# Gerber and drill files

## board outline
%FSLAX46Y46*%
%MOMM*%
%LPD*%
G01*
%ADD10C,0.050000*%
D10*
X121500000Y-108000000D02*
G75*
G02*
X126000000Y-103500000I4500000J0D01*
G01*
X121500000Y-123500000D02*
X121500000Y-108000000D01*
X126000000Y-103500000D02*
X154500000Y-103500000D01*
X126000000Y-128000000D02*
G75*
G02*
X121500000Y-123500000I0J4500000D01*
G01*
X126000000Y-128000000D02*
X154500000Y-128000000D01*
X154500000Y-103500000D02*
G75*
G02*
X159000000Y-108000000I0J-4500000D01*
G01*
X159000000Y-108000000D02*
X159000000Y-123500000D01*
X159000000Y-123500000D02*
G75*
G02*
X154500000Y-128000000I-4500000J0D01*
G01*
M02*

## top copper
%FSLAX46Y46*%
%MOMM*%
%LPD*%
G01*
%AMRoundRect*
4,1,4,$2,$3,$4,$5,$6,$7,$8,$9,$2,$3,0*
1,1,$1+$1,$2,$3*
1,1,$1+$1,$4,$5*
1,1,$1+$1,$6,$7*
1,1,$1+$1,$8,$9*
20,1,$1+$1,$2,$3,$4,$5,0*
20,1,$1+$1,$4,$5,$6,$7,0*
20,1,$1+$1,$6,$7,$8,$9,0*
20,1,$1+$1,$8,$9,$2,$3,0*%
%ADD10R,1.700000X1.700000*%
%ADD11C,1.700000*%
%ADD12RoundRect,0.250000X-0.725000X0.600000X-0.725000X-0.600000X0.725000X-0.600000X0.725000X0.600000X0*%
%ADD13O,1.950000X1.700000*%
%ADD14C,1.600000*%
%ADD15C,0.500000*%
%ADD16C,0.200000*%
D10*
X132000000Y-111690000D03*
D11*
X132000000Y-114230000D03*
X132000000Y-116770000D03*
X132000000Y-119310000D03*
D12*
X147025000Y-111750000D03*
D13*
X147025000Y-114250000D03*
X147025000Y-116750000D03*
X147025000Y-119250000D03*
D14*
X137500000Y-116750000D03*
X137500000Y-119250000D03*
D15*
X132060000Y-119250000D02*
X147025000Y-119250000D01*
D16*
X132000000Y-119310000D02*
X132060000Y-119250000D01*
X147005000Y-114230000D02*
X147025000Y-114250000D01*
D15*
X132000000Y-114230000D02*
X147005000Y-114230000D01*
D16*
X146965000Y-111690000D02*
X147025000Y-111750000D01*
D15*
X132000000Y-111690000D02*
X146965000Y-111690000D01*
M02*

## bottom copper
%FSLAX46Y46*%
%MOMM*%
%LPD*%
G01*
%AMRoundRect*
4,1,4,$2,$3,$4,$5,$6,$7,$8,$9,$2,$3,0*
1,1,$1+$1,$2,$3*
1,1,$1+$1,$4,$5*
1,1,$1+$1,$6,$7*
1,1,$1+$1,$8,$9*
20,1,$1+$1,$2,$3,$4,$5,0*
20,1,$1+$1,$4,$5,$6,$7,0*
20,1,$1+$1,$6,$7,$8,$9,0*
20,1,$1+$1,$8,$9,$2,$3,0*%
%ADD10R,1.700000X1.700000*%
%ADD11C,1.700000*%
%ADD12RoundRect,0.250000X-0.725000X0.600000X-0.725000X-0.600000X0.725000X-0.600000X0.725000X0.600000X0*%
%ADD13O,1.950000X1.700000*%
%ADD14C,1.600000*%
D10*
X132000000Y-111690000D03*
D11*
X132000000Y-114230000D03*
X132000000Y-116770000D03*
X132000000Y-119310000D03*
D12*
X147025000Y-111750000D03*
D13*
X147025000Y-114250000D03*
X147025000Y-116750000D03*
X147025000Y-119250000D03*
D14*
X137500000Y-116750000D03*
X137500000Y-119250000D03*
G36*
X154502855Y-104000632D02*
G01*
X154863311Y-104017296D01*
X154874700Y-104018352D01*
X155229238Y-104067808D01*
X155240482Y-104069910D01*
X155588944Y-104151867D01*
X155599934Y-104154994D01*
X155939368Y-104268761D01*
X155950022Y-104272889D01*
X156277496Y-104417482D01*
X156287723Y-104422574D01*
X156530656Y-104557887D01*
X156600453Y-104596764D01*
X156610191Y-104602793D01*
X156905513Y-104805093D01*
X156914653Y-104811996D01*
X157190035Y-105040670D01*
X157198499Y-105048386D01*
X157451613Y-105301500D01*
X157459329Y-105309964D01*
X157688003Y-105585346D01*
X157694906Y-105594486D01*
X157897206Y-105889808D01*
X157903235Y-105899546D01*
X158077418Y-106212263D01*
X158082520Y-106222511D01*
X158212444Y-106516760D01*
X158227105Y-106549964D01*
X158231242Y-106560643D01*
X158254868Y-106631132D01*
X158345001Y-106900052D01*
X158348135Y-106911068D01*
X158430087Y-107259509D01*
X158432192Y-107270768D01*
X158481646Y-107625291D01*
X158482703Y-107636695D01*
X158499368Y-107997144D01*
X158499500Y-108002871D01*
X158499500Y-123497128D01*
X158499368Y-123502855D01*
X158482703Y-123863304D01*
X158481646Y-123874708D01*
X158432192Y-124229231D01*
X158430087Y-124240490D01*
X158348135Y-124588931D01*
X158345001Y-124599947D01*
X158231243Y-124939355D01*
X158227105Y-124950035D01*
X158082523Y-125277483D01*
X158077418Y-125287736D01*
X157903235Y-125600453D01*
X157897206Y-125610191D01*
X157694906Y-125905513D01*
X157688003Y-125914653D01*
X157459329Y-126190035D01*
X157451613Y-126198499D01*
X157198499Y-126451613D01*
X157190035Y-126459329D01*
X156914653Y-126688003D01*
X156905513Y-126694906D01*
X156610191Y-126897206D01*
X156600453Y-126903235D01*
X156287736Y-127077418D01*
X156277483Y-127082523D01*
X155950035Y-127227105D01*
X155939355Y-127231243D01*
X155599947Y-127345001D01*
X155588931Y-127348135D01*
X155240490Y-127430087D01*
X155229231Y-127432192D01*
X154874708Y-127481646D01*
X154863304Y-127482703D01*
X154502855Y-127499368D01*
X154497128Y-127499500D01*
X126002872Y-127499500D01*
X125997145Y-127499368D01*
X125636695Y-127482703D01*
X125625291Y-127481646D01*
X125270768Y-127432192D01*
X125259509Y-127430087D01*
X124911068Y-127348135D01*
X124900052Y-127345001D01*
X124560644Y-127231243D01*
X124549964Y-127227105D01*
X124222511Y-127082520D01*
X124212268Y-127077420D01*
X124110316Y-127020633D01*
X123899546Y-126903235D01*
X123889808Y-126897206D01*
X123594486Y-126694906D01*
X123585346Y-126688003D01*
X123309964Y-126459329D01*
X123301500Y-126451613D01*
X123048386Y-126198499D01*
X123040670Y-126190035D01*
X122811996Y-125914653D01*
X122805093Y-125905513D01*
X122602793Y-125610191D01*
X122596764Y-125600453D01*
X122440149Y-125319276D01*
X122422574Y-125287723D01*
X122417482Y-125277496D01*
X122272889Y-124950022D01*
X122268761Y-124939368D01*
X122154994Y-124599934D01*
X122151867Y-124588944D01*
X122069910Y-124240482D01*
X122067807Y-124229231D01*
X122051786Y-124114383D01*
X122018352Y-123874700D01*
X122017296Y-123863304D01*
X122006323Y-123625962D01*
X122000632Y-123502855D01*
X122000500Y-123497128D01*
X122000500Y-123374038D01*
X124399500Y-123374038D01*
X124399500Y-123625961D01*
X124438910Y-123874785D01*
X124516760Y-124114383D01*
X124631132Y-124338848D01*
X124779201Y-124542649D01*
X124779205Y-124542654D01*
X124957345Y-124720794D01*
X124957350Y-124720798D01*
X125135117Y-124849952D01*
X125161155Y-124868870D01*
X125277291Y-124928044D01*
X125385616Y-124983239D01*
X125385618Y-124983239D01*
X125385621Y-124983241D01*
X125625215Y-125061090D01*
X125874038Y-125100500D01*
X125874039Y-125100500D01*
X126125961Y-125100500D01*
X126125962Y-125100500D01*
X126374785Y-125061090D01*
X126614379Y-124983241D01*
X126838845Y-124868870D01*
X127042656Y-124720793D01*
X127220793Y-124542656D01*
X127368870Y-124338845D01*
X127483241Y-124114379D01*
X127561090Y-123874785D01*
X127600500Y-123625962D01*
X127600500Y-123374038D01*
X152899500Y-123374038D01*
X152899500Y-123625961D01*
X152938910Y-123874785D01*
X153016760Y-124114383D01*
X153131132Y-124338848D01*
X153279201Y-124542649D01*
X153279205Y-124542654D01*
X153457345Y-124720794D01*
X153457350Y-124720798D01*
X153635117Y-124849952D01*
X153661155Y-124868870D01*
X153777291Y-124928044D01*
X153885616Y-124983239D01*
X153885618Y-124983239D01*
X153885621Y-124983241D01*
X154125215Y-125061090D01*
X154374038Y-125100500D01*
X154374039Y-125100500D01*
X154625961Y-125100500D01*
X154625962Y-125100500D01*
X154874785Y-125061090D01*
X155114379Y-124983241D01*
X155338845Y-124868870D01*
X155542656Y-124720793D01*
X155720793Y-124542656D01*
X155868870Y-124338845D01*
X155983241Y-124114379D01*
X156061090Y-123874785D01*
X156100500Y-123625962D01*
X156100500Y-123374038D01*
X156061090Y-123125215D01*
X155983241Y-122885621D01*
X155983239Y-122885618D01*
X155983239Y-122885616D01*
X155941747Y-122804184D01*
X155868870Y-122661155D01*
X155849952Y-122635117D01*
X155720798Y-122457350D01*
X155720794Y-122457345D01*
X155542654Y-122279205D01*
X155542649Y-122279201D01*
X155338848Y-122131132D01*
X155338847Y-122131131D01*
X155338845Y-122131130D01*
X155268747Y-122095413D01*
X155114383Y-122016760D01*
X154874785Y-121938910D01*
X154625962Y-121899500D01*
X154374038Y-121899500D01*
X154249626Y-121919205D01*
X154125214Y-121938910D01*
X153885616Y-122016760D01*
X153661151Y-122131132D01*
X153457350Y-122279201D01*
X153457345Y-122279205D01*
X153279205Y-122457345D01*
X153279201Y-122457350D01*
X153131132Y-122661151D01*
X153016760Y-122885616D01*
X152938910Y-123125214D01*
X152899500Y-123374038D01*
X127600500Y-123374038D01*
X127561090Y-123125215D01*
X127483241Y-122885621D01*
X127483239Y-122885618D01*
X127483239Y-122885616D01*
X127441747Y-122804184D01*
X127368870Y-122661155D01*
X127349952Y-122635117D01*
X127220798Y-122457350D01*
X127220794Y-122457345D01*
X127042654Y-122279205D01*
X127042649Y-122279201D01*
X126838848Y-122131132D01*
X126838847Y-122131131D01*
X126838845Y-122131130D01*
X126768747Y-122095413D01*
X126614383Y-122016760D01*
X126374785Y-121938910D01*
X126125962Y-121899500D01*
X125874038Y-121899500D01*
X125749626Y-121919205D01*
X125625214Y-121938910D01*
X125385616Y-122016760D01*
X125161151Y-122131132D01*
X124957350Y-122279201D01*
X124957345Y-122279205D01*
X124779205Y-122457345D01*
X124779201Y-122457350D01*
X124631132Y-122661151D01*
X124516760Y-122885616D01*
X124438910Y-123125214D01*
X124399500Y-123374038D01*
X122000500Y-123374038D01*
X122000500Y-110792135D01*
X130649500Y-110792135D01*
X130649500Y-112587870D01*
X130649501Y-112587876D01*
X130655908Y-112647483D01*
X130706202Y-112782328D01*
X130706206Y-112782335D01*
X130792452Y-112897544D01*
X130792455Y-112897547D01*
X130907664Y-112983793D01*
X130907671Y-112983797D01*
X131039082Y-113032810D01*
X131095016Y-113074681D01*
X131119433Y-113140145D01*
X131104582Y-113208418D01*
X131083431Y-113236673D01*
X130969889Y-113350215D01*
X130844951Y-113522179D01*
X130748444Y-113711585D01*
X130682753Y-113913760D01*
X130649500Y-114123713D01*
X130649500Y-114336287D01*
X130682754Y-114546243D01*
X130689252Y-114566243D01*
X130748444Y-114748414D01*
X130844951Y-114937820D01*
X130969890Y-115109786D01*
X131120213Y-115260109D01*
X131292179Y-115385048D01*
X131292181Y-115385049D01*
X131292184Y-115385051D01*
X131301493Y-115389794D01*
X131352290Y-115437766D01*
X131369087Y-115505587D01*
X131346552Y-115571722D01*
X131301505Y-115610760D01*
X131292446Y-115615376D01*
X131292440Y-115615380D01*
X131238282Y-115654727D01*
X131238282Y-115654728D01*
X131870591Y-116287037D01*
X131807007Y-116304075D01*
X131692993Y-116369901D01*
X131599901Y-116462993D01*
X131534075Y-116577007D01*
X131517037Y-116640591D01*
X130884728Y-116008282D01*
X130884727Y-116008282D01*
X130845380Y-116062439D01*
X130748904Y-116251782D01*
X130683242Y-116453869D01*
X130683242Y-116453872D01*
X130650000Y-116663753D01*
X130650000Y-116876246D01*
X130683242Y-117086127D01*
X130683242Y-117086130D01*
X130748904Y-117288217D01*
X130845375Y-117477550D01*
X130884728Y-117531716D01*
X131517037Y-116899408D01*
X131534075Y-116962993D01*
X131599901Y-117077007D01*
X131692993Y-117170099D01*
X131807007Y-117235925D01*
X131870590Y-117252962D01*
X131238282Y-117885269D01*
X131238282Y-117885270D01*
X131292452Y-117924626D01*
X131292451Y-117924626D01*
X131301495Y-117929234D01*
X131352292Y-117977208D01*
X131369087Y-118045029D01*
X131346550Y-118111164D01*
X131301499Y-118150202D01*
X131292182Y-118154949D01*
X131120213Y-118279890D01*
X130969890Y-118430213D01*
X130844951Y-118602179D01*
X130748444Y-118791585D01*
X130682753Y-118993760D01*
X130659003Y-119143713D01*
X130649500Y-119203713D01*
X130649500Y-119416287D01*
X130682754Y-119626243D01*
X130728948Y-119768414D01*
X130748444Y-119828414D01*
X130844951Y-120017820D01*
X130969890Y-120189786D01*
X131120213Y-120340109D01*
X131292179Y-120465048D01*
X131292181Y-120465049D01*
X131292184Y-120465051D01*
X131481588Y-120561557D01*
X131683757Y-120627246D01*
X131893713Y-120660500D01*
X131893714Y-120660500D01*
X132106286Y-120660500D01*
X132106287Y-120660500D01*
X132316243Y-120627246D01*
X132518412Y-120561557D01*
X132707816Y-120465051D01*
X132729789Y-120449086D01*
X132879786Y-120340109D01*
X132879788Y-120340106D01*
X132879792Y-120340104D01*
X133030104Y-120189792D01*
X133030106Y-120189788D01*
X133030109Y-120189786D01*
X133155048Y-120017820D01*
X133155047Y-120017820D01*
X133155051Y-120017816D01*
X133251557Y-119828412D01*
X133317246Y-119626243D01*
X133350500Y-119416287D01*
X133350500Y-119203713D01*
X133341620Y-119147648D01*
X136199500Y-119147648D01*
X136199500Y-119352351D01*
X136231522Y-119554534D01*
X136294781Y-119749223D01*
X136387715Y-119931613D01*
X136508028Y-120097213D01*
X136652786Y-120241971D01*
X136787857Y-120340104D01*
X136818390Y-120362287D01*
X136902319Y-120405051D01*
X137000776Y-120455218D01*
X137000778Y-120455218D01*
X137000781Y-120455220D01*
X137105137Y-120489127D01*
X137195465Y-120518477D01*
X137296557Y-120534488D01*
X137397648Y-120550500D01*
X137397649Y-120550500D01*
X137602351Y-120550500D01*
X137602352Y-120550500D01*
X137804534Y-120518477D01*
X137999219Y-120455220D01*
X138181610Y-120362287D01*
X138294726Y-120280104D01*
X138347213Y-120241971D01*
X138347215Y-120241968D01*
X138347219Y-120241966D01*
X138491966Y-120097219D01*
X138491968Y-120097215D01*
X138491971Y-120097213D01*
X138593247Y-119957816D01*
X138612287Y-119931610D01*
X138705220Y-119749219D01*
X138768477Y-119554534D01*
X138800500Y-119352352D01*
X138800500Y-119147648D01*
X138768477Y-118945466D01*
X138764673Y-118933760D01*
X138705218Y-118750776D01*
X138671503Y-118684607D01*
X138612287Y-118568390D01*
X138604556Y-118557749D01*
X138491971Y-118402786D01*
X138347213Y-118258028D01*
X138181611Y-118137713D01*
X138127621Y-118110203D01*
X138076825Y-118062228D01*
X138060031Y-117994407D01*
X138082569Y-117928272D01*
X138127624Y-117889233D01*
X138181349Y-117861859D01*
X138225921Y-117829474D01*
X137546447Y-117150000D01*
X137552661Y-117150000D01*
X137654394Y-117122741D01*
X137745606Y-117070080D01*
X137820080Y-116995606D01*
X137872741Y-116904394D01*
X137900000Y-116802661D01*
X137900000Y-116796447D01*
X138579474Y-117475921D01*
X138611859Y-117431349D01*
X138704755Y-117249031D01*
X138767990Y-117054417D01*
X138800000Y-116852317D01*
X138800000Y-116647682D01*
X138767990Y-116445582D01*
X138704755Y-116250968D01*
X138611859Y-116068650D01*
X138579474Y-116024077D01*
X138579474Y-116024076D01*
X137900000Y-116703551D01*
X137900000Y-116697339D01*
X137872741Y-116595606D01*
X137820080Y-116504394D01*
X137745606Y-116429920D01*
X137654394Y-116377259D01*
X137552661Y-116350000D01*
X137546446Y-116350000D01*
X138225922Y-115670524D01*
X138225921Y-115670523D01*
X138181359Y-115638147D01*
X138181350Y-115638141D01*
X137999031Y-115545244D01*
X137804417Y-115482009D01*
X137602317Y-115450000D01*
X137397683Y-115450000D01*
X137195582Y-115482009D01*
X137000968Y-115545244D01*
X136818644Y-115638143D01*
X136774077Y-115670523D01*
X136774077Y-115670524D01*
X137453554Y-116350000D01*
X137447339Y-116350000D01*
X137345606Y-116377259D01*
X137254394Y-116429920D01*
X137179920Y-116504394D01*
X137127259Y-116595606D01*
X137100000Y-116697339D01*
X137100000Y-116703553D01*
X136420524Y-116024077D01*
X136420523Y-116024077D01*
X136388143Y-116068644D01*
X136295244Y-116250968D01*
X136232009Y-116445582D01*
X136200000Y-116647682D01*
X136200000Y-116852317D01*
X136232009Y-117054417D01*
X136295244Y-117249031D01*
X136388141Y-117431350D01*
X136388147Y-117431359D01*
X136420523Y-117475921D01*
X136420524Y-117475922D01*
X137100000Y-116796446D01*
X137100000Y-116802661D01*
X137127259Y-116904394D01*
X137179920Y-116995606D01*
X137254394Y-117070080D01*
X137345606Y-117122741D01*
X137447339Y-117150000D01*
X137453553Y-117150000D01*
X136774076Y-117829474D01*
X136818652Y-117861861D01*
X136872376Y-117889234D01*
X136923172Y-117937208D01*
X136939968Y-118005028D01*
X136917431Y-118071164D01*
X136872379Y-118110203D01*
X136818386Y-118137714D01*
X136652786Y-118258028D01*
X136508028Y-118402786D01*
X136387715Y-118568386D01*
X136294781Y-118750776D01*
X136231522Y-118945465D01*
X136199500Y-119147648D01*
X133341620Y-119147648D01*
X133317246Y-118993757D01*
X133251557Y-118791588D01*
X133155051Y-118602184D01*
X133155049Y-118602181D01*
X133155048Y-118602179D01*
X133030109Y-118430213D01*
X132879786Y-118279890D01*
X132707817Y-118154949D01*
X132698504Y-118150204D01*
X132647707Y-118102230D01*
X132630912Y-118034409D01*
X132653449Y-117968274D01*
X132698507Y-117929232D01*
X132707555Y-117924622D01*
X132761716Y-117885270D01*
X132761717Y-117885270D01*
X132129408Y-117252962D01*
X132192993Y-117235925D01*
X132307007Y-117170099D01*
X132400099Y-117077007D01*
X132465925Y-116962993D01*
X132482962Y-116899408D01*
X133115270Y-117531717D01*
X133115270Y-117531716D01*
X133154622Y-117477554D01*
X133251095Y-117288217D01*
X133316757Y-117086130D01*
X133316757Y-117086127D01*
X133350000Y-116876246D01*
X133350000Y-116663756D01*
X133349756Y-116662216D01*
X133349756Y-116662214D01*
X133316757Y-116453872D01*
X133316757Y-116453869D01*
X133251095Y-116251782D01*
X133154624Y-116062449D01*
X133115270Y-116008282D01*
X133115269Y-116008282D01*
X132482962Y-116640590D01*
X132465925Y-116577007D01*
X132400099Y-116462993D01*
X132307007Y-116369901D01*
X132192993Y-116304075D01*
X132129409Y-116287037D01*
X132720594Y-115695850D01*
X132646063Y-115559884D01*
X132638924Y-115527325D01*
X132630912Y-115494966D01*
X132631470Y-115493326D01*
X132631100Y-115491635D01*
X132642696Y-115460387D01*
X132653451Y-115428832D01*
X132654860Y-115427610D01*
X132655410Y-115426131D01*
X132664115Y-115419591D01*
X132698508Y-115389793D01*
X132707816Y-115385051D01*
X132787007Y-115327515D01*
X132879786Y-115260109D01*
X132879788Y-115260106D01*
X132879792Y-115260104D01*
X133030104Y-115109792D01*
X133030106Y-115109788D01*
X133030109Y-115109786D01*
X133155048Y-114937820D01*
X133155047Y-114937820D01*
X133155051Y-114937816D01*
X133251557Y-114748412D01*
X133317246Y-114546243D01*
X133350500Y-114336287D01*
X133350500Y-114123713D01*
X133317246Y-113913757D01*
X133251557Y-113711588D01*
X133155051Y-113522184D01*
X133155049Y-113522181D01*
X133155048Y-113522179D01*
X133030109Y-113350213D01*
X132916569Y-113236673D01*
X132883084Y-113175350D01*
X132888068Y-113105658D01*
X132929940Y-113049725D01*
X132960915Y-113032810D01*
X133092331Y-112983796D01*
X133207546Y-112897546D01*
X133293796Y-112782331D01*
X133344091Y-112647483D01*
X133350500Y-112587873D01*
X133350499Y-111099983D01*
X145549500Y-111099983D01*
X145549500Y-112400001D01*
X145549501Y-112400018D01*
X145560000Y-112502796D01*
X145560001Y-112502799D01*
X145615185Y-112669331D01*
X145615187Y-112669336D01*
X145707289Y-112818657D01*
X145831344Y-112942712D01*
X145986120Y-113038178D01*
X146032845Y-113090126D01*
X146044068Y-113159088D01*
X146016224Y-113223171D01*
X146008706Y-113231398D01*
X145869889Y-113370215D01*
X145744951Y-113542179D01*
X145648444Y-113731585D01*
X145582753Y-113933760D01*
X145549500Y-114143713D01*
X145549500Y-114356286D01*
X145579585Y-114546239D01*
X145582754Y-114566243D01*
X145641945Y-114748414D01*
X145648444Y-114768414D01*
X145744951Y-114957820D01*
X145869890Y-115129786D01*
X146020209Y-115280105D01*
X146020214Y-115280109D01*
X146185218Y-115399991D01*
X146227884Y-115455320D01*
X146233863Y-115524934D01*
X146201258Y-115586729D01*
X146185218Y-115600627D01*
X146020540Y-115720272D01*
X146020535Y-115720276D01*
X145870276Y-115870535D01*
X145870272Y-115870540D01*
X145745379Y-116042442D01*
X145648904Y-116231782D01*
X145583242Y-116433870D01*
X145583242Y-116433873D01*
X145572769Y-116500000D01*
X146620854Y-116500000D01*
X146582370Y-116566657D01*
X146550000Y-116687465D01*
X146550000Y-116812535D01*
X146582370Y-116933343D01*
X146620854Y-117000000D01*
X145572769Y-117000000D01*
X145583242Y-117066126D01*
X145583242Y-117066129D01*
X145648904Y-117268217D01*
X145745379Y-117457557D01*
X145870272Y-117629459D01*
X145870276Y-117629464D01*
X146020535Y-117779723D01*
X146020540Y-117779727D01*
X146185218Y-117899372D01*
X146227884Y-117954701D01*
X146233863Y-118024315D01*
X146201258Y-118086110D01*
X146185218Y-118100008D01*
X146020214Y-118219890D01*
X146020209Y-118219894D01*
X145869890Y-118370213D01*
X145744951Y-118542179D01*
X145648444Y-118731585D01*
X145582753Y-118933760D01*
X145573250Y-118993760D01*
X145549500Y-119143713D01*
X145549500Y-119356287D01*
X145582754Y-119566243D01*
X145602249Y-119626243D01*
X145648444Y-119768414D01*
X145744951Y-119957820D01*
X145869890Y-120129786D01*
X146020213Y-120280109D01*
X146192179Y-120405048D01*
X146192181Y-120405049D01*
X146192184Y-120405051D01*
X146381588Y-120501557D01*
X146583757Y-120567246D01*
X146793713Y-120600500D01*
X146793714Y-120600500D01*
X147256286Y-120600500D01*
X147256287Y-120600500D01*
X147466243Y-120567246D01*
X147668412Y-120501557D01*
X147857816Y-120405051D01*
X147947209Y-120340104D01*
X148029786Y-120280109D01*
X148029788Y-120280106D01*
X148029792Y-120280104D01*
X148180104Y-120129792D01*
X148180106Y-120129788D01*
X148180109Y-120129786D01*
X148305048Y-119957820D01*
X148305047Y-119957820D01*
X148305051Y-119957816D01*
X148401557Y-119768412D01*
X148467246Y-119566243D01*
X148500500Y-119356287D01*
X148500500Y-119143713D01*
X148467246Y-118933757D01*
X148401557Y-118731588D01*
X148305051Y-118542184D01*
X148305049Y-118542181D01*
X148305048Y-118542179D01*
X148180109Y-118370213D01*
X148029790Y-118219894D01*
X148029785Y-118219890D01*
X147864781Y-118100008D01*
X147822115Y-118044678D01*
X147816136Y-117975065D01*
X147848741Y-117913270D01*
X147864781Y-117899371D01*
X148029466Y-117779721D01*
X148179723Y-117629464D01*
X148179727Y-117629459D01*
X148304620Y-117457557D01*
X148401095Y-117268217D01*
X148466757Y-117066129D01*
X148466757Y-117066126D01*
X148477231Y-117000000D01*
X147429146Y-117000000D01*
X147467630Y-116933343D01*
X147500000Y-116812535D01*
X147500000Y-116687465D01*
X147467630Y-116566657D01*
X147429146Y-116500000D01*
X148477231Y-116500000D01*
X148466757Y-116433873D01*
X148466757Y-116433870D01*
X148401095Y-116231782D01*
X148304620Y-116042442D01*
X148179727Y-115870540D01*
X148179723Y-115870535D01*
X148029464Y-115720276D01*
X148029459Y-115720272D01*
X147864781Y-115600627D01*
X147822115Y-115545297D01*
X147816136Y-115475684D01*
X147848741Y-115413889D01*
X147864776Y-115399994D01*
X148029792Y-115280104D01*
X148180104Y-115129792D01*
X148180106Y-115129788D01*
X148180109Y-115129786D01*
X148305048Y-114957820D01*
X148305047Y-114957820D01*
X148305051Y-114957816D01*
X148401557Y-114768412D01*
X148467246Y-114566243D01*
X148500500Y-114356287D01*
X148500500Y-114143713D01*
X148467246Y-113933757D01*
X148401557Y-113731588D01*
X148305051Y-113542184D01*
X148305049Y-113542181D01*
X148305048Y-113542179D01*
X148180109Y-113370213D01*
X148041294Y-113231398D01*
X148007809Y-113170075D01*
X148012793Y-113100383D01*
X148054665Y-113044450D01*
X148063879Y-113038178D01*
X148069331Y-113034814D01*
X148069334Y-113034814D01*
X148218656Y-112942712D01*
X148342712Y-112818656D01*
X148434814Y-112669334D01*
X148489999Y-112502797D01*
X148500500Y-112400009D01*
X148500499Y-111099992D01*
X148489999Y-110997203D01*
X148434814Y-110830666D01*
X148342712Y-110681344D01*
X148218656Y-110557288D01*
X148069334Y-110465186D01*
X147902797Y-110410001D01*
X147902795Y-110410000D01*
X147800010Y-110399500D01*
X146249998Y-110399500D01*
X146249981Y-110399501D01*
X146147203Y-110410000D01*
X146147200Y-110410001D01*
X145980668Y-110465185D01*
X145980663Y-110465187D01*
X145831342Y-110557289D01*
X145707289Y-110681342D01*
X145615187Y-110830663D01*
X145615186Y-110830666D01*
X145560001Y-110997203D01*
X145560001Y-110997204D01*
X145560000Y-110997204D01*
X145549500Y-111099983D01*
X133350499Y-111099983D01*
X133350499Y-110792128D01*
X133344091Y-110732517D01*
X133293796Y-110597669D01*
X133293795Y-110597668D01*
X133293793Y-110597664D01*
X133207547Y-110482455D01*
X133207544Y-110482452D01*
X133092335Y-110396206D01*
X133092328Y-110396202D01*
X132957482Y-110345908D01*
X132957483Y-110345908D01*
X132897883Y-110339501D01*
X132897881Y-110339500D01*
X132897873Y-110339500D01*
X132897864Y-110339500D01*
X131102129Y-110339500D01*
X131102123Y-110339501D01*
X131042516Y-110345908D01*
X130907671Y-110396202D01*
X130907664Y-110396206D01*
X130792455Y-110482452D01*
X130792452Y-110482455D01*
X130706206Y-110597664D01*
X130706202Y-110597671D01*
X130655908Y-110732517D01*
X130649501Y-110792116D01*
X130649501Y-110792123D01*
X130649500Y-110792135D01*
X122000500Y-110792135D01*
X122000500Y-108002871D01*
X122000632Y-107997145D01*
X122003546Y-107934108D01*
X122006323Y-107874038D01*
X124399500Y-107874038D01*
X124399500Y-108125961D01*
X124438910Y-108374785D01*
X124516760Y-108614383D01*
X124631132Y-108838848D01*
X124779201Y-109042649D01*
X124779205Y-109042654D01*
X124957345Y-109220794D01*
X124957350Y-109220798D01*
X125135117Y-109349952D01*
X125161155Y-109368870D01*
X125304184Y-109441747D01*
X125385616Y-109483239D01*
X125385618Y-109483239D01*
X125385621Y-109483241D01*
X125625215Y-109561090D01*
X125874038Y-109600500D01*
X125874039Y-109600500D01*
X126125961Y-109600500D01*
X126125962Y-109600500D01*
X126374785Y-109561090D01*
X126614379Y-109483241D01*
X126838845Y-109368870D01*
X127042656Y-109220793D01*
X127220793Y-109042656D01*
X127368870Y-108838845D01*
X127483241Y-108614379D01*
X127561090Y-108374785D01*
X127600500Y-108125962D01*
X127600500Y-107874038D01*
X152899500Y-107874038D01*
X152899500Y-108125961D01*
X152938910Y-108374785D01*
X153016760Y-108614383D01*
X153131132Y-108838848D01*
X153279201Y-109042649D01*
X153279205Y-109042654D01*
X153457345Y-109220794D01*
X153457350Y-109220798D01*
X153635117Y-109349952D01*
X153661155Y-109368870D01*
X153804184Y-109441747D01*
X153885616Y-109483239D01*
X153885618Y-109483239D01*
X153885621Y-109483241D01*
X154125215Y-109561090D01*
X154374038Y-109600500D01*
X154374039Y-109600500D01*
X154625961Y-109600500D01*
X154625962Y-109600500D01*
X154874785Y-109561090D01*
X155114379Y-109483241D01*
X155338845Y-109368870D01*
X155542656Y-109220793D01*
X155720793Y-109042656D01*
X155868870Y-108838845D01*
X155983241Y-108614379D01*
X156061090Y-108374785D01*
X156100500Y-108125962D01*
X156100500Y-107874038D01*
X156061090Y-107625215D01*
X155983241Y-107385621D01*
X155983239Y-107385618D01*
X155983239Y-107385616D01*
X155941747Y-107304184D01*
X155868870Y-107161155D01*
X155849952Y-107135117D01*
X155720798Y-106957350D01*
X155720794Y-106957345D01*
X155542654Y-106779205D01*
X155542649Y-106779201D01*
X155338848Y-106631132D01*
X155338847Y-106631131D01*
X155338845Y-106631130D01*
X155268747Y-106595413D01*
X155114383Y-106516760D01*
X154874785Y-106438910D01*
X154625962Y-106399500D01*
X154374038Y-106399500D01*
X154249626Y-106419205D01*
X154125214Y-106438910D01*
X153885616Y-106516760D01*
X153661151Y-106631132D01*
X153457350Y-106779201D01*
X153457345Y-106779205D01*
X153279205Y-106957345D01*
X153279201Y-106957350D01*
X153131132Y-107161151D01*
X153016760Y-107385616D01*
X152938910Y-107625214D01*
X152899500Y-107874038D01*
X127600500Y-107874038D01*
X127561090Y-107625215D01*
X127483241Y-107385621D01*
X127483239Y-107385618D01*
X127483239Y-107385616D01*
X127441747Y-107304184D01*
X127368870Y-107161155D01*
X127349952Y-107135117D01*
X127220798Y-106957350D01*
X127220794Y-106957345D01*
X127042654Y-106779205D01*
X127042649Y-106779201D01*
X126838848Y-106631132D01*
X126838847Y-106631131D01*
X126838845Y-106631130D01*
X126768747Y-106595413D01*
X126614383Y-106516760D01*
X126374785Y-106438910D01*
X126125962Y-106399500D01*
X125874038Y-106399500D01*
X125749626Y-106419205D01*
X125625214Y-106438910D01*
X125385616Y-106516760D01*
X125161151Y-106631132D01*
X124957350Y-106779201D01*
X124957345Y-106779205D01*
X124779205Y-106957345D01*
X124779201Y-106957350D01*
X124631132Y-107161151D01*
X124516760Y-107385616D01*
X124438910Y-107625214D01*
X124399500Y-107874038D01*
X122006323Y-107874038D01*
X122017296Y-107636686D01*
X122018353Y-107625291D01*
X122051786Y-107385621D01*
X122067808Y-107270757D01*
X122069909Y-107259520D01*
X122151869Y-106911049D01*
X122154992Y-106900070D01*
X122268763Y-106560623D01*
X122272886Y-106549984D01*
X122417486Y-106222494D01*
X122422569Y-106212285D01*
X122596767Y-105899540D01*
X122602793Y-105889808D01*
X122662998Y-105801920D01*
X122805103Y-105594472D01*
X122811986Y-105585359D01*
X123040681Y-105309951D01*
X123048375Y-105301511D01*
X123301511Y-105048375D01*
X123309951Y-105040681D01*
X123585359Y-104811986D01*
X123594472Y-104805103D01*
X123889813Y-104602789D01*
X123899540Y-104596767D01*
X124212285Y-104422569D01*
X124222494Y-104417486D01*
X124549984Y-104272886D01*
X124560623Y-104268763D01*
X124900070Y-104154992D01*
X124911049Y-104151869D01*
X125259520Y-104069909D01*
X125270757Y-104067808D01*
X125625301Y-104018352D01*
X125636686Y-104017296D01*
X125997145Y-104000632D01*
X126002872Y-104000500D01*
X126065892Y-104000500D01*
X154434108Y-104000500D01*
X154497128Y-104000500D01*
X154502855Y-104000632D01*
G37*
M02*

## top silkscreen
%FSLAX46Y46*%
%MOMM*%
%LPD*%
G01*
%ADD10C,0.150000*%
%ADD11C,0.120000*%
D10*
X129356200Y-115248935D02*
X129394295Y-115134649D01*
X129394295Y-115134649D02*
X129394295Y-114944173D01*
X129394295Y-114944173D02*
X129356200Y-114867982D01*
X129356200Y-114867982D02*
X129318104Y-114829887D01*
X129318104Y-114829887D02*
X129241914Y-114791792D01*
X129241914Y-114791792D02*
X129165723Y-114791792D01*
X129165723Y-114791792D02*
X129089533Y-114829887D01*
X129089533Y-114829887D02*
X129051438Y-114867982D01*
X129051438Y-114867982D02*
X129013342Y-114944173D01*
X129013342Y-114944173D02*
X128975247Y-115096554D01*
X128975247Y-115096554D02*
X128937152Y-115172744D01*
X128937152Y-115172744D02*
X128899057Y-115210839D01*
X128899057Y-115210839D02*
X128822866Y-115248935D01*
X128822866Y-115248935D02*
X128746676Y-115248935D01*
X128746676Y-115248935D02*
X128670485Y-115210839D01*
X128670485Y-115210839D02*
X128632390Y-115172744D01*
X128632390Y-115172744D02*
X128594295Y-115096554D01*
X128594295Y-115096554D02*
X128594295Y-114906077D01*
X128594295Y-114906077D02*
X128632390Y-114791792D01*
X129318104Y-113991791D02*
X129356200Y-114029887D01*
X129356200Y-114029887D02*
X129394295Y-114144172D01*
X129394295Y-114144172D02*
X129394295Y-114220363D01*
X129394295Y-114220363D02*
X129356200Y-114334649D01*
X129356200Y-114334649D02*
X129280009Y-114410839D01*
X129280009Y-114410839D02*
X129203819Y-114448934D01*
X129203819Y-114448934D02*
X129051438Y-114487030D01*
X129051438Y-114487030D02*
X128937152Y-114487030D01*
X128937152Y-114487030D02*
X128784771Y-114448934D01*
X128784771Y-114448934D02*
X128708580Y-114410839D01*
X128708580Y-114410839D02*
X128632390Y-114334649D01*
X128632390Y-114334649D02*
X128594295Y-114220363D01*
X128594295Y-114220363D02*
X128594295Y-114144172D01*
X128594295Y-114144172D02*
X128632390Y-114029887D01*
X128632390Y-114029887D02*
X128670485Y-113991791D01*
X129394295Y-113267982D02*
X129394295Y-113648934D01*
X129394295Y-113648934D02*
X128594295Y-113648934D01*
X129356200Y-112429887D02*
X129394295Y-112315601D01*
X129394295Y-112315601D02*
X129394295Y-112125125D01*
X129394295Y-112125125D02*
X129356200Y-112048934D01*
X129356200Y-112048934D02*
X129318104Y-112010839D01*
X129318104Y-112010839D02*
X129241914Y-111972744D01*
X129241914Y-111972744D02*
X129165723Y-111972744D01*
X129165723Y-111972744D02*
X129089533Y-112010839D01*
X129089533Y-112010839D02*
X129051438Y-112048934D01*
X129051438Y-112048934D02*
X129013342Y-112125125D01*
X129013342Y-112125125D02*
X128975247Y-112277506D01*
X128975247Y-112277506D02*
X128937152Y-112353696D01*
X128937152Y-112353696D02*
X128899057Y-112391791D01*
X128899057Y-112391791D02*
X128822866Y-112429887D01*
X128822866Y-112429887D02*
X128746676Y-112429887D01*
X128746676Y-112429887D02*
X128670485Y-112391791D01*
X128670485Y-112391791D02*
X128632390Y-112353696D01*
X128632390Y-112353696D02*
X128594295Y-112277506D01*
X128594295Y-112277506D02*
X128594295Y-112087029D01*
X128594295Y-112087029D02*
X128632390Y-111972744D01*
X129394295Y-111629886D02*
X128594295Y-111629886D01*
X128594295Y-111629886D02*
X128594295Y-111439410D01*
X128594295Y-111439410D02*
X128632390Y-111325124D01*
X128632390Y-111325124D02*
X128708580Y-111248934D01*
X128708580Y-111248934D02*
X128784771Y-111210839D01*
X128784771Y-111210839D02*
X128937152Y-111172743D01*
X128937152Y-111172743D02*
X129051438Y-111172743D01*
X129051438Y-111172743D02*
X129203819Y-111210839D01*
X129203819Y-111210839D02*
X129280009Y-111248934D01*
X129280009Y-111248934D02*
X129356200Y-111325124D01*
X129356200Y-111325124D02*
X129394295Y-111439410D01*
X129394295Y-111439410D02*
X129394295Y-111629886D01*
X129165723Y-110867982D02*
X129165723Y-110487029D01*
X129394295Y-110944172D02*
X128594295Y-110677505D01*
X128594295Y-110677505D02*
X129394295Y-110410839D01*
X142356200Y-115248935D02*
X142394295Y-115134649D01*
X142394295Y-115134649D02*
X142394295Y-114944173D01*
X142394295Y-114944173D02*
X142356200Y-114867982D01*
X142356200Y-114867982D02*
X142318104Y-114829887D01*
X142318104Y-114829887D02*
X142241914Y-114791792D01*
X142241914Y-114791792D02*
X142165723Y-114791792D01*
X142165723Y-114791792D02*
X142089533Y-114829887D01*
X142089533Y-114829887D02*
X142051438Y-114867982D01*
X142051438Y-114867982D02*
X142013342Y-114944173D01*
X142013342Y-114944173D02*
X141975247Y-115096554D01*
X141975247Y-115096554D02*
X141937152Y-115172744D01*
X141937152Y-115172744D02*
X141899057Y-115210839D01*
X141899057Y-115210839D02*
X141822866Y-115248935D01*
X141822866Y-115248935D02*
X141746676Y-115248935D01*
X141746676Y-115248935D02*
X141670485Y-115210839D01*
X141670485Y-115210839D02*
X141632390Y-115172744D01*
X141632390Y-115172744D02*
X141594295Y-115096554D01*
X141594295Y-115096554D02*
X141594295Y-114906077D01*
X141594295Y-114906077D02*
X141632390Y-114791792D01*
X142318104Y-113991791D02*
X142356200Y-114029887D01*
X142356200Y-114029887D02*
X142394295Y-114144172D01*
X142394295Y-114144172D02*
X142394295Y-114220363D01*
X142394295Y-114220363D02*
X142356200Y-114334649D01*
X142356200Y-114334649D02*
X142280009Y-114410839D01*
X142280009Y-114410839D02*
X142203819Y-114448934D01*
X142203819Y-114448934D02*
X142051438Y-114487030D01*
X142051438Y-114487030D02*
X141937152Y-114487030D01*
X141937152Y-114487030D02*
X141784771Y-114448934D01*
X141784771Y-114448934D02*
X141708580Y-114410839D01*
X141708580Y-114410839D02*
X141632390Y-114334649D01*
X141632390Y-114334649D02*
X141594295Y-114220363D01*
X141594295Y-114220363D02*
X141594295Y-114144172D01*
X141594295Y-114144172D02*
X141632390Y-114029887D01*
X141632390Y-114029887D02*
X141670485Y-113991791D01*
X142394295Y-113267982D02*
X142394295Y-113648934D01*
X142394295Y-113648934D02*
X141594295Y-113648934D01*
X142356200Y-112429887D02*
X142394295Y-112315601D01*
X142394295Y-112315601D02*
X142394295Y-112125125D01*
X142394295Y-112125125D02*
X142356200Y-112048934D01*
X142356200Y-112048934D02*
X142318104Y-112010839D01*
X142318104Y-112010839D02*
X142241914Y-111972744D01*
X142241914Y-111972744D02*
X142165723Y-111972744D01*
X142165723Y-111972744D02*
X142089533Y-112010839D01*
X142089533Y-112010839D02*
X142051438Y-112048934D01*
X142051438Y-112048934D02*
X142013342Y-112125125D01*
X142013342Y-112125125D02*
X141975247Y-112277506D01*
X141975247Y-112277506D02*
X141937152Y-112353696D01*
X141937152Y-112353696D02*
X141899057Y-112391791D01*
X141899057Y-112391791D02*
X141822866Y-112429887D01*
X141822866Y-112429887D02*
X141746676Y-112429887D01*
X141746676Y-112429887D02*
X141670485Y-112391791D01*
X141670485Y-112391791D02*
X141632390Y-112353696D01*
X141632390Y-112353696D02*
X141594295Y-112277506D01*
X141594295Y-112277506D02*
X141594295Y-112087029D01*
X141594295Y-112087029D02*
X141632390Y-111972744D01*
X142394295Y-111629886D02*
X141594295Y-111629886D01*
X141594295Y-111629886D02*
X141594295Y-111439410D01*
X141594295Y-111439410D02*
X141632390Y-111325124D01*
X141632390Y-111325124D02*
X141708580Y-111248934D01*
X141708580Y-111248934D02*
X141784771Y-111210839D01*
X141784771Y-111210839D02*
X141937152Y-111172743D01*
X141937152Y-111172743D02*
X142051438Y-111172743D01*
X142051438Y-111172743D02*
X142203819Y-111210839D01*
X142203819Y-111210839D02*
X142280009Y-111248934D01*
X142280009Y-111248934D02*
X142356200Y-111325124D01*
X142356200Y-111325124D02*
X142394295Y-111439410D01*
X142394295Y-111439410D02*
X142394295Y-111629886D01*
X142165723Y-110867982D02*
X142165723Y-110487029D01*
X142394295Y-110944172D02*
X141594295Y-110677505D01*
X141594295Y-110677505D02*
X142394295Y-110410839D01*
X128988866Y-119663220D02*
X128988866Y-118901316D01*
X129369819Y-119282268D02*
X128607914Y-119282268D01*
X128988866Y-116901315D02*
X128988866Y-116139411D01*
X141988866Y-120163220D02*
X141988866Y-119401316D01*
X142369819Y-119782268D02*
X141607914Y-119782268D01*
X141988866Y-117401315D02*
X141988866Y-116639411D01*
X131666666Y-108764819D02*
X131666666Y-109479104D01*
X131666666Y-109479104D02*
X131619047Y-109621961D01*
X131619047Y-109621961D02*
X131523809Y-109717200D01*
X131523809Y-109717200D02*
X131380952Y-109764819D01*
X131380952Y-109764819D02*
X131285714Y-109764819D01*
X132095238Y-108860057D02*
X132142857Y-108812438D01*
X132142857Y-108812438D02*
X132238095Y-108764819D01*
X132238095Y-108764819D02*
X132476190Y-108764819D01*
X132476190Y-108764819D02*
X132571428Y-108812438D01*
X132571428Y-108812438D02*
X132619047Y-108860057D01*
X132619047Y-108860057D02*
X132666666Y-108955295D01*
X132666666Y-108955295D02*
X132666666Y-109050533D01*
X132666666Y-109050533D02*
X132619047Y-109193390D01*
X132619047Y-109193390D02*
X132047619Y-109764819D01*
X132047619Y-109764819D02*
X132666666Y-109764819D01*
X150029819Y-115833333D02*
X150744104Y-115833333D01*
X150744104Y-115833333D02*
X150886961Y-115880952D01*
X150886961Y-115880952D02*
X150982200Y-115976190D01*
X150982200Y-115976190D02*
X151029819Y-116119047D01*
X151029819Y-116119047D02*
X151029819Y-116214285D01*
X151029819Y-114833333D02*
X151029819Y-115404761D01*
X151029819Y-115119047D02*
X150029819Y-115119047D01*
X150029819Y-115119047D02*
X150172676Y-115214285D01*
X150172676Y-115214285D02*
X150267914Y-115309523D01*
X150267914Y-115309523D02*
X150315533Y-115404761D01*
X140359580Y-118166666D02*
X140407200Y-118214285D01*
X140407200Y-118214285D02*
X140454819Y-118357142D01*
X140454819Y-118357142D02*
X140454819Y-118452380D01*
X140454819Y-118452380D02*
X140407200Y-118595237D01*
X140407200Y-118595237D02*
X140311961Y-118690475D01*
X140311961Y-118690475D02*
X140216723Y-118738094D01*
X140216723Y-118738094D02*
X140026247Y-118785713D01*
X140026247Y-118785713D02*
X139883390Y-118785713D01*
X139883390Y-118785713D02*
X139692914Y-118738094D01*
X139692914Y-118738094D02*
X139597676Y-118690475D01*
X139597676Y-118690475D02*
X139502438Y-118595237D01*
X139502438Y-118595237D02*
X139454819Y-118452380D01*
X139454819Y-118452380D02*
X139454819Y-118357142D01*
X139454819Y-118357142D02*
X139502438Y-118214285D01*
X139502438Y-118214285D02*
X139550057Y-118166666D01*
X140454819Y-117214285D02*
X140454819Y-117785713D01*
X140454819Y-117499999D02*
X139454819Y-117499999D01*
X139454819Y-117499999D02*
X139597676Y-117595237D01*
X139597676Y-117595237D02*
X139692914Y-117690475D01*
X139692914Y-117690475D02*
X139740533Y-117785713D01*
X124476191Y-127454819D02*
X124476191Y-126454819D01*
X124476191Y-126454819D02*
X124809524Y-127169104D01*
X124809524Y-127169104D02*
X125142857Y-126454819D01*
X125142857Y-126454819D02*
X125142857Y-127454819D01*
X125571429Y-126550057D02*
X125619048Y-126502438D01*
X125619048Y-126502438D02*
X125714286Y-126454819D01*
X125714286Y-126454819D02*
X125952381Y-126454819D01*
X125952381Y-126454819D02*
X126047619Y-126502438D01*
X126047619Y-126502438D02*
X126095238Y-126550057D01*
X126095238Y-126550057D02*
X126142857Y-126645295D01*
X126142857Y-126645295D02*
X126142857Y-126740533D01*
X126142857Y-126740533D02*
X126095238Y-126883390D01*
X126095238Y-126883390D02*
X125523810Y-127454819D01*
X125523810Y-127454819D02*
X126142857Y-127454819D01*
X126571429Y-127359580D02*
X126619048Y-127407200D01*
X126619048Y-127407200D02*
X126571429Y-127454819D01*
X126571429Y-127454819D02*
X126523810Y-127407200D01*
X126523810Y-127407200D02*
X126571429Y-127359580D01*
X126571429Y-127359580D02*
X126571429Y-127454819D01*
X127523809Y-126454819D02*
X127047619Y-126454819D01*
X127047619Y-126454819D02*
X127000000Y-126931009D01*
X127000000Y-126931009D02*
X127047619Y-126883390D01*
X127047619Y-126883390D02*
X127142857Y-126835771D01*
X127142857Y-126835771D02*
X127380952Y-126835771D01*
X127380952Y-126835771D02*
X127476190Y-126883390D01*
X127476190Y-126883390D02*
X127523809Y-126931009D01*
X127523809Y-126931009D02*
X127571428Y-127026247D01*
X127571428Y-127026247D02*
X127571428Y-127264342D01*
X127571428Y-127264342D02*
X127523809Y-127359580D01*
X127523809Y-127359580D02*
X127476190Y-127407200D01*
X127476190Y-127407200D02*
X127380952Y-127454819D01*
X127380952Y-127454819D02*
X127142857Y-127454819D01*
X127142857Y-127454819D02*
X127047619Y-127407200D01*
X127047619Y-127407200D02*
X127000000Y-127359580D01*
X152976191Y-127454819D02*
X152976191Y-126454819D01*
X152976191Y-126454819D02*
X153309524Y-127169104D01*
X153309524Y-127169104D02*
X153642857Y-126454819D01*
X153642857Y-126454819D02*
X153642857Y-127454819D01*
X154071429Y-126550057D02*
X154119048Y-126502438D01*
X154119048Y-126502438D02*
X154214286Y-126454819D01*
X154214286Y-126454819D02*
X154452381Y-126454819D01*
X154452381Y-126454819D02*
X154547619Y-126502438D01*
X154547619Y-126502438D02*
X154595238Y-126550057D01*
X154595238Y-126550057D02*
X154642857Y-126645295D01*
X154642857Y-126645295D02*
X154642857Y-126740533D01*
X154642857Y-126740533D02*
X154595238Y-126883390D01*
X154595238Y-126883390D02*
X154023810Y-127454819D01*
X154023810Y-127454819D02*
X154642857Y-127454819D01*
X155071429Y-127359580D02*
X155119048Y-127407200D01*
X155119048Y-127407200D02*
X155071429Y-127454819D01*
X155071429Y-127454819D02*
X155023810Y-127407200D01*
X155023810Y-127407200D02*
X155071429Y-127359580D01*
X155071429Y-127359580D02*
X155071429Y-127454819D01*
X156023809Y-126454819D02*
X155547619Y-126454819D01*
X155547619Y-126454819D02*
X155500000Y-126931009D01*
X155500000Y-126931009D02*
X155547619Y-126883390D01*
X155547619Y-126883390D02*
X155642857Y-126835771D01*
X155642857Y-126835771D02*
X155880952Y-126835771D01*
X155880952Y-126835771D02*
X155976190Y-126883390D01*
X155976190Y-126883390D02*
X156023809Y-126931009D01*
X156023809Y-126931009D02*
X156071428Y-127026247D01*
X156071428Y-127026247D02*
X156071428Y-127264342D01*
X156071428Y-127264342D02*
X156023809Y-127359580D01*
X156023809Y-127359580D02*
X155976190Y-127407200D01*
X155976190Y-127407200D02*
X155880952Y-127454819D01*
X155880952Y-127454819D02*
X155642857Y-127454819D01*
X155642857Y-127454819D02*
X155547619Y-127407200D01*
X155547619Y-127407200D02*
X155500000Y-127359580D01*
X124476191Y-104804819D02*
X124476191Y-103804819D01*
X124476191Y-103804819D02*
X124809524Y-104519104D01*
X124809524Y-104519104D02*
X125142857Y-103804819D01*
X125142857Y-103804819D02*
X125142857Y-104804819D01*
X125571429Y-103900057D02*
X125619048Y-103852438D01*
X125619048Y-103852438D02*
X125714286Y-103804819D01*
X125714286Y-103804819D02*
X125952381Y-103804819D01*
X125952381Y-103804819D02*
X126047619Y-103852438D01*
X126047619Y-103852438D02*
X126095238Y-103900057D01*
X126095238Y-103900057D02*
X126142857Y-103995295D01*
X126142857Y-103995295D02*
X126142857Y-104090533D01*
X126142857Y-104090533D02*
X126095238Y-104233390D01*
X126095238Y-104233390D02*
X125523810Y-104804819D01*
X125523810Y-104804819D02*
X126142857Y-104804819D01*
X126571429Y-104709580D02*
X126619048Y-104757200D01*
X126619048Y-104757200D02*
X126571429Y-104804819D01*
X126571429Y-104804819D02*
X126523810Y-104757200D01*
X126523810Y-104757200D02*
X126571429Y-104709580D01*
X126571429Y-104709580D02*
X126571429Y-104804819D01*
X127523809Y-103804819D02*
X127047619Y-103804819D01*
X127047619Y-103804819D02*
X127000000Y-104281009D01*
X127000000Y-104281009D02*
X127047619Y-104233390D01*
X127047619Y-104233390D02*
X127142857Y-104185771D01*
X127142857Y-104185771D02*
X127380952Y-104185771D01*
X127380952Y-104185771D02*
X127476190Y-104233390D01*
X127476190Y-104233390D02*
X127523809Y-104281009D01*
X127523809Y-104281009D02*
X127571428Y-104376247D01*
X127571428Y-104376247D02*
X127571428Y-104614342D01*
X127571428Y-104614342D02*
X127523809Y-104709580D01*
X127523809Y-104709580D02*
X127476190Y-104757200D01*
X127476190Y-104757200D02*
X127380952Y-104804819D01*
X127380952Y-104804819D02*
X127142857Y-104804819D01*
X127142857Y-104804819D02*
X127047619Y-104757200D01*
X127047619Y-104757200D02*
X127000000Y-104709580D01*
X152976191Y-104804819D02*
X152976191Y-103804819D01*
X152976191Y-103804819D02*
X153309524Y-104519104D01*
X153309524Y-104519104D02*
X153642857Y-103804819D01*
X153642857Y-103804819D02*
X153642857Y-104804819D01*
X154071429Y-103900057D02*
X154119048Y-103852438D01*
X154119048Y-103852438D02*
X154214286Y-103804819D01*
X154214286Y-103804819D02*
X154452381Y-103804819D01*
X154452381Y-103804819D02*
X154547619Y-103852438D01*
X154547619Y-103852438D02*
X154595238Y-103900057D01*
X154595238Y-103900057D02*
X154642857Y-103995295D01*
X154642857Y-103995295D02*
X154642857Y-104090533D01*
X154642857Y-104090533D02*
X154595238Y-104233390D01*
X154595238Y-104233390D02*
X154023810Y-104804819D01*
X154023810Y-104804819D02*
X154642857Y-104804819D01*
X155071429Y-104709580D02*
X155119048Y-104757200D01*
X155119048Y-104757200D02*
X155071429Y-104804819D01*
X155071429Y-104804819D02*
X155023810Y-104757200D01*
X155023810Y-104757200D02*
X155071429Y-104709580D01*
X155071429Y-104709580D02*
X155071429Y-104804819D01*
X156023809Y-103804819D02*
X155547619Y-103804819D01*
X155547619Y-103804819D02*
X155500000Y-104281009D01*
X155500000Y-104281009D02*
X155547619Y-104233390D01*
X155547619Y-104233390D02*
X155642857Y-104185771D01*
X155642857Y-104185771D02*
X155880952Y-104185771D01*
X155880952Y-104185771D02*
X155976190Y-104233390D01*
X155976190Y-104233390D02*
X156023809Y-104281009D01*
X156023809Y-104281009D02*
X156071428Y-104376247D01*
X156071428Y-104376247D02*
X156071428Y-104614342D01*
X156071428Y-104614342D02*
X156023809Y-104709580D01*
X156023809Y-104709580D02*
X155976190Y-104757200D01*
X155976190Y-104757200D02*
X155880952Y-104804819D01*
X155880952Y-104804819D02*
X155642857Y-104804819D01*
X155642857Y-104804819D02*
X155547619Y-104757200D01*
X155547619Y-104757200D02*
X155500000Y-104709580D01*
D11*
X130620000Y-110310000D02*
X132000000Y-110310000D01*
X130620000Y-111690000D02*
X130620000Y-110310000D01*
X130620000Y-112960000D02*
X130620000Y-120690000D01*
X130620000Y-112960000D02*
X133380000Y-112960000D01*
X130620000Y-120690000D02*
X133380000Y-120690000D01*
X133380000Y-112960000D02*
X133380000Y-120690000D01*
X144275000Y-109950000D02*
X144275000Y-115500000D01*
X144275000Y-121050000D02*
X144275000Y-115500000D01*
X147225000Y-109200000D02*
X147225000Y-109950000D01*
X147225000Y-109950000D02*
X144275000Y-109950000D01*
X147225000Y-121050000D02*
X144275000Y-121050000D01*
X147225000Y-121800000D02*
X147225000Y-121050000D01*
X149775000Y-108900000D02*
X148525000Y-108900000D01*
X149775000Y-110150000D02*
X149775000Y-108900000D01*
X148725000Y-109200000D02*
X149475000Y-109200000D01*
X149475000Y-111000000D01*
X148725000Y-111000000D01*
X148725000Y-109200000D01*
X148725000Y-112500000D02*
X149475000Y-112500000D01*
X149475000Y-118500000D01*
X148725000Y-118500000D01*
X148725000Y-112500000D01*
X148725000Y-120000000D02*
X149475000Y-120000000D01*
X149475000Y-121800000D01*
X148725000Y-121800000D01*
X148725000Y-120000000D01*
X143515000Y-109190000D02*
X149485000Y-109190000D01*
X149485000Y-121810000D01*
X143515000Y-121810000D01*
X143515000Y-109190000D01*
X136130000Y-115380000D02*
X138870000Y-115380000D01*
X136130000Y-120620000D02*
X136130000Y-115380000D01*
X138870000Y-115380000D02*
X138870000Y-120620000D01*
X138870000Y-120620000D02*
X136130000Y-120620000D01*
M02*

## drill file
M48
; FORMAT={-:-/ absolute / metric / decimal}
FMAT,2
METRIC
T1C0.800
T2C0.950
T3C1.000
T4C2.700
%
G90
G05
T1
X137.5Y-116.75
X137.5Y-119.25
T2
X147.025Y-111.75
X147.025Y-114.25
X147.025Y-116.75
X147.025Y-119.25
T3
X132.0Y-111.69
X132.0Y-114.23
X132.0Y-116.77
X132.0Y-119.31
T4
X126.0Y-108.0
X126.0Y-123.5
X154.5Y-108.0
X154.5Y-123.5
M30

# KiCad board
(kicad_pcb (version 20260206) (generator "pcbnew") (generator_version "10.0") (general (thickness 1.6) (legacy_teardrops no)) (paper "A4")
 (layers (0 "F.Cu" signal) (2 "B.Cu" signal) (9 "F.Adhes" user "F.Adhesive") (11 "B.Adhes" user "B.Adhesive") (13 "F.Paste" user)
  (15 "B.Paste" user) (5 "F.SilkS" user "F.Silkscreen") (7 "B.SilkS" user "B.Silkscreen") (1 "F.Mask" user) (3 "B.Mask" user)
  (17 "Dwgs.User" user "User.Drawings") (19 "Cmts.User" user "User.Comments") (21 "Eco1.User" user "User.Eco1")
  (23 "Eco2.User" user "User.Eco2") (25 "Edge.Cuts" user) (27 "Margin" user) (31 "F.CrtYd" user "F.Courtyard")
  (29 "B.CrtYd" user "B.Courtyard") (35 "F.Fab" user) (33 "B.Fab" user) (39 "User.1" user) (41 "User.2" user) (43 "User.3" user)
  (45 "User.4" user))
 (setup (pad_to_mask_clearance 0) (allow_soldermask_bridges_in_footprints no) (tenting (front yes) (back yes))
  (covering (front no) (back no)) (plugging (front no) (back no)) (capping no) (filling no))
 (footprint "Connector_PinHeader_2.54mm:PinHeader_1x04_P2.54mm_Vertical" (layer "F.Cu") (at 132 111.69)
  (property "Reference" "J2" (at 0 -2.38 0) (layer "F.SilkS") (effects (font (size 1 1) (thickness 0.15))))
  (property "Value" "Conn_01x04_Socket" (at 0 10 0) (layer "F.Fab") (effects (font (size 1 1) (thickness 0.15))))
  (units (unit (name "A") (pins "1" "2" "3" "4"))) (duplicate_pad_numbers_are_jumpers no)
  (fp_line (start -1.38 -1.38) (end 0 -1.38) (stroke (width 0.12) (type solid)) (layer "F.SilkS"))
  (fp_line (start -1.38 0) (end -1.38 -1.38) (stroke (width 0.12) (type solid)) (layer "F.SilkS"))
  (fp_line (start -1.38 1.27) (end -1.38 9) (stroke (width 0.12) (type solid)) (layer "F.SilkS"))
  (fp_line (start -1.38 1.27) (end 1.38 1.27) (stroke (width 0.12) (type solid)) (layer "F.SilkS"))
  (fp_line (start -1.38 9) (end 1.38 9) (stroke (width 0.12) (type solid)) (layer "F.SilkS"))
  (fp_line (start 1.38 1.27) (end 1.38 9) (stroke (width 0.12) (type solid)) (layer "F.SilkS"))
  (pad "1" thru_hole rect (at 0 0) (size 1.7 1.7) (drill 1) (layers "*.Cu" "*.Mask") (remove_unused_layers no) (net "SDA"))
  (pad "2" thru_hole circle (at 0 2.54) (size 1.7 1.7) (drill 1) (layers "*.Cu" "*.Mask") (remove_unused_layers no) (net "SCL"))
  (pad "3" thru_hole circle (at 0 5.08) (size 1.7 1.7) (drill 1) (layers "*.Cu" "*.Mask") (remove_unused_layers no) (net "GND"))
  (pad "4" thru_hole circle (at 0 7.62) (size 1.7 1.7) (drill 1) (layers "*.Cu" "*.Mask") (remove_unused_layers no) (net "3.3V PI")))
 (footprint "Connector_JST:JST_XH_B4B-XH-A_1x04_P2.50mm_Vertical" (layer "F.Cu") (at 147.025 111.75 -90)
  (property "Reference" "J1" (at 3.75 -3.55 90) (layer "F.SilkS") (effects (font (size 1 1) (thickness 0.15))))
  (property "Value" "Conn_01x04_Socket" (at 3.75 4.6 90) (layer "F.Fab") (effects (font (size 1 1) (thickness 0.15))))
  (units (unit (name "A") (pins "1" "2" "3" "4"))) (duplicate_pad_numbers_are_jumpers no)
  (fp_line (start -1.8 2.75) (end 3.75 2.75) (stroke (width 0.12) (type solid)) (layer "F.SilkS"))
  (fp_line (start 9.3 2.75) (end 3.75 2.75) (stroke (width 0.12) (type solid)) (layer "F.SilkS"))
  (fp_line (start -2.55 -0.2) (end -1.8 -0.2) (stroke (width 0.12) (type solid)) (layer "F.SilkS"))
  (fp_line (start -1.8 -0.2) (end -1.8 2.75) (stroke (width 0.12) (type solid)) (layer "F.SilkS"))
  (fp_line (start 9.3 -0.2) (end 9.3 2.75) (stroke (width 0.12) (type solid)) (layer "F.SilkS"))
  (fp_line (start 10.05 -0.2) (end 9.3 -0.2) (stroke (width 0.12) (type solid)) (layer "F.SilkS"))
  (fp_line (start -2.85 -2.75) (end -2.85 -1.5) (stroke (width 0.12) (type solid)) (layer "F.SilkS"))
  (fp_line (start -1.6 -2.75) (end -2.85 -2.75) (stroke (width 0.12) (type solid)) (layer "F.SilkS"))
  (fp_rect (start -2.55 -2.45) (end -0.75 -1.7) (stroke (width 0.12) (type solid)) (fill no) (layer "F.SilkS"))
  (fp_rect (start 0.75 -2.45) (end 6.75 -1.7) (stroke (width 0.12) (type solid)) (fill no) (layer "F.SilkS"))
  (fp_rect (start 8.25 -2.45) (end 10.05 -1.7) (stroke (width 0.12) (type solid)) (fill no) (layer "F.SilkS"))
  (fp_rect (start -2.56 -2.46) (end 10.06 3.51) (stroke (width 0.12) (type solid)) (fill no) (layer "F.SilkS"))
  (pad "1" thru_hole roundrect (at 0 0 270) (size 1.7 1.95) (drill 0.95) (layers "*.Cu" "*.Mask") (remove_unused_layers no)
   (roundrect_rratio 0.147059) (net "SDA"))
  (pad "2" thru_hole oval (at 2.5 0 270) (size 1.7 1.95) (drill 0.95) (layers "*.Cu" "*.Mask") (remove_unused_layers no) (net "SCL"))
  (pad "3" thru_hole oval (at 5 0 270) (size 1.7 1.95) (drill 0.95) (layers "*.Cu" "*.Mask") (remove_unused_layers no) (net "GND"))
  (pad "4" thru_hole oval (at 7.5 0 270) (size 1.7 1.95) (drill 0.95) (layers "*.Cu" "*.Mask") (remove_unused_layers no) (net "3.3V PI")))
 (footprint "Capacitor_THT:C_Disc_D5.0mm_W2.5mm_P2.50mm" (layer "F.Cu") (at 137.5 116.75 -90)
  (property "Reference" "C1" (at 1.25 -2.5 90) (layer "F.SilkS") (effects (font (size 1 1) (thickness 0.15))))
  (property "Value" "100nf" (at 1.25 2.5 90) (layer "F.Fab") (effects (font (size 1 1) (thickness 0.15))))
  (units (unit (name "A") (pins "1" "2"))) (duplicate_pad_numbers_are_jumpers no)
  (fp_line (start -1.37 1.37) (end -1.37 -1.37) (stroke (width 0.12) (type solid)) (layer "F.SilkS"))
  (fp_line (start 3.87 1.37) (end -1.37 1.37) (stroke (width 0.12) (type solid)) (layer "F.SilkS"))
  (fp_line (start -1.37 -1.37) (end 3.87 -1.37) (stroke (width 0.12) (type solid)) (layer "F.SilkS"))
  (fp_line (start 3.87 -1.37) (end 3.87 1.37) (stroke (width 0.12) (type solid)) (layer "F.SilkS"))
  (pad "1" thru_hole circle (at 0 0 270) (size 1.6 1.6) (drill 0.8) (layers "*.Cu" "*.Mask") (remove_unused_layers no) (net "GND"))
  (pad "2" thru_hole circle (at 2.5 0 270) (size 1.6 1.6) (drill 0.8) (layers "*.Cu" "*.Mask") (remove_unused_layers no) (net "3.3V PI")))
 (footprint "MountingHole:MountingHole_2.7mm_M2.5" (layer "F.Cu") (at 126 123.5)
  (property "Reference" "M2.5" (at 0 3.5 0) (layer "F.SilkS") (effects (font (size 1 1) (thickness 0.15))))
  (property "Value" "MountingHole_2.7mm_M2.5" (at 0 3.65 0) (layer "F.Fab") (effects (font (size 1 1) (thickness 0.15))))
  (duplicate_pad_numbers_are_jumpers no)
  (pad "" np_thru_hole circle (at 0 0) (size 2.7 2.7) (drill 2.7) (layers "*.Cu" "*.Mask")))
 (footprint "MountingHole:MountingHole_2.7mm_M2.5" (layer "F.Cu") (at 154.5 123.5)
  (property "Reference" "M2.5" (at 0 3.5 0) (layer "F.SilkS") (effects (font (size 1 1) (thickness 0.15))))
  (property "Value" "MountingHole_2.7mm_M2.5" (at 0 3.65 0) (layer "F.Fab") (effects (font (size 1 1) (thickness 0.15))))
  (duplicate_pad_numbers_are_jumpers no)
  (pad "" np_thru_hole circle (at 0 0) (size 2.7 2.7) (drill 2.7) (layers "*.Cu" "*.Mask")))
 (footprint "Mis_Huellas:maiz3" (layer "F.Cu") (at 141 115.5)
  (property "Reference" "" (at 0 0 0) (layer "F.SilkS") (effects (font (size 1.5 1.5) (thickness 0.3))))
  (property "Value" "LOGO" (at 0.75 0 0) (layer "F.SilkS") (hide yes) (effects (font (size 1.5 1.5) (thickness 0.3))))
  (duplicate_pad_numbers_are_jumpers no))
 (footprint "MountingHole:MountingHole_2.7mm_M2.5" (layer "F.Cu") (at 126 108)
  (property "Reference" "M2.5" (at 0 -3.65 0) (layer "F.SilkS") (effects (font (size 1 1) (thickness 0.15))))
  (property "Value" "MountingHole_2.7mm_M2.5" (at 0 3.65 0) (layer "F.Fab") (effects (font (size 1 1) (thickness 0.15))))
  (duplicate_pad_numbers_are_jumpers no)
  (pad "" np_thru_hole circle (at 0 0) (size 2.7 2.7) (drill 2.7) (layers "*.Cu" "*.Mask")))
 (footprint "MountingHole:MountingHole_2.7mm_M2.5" (layer "F.Cu") (at 154.5 108)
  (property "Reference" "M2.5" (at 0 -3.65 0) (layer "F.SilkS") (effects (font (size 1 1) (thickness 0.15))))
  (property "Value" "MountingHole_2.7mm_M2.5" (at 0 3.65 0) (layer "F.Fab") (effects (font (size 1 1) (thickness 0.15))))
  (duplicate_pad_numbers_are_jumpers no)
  (pad "" np_thru_hole circle (at 0 0) (size 2.7 2.7) (drill 2.7) (layers "*.Cu" "*.Mask")))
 (gr_arc (start 121.5 108) (mid 122.818019 104.818019) (end 126 103.5) (stroke (width 0.05) (type default)) (layer "Edge.Cuts"))
 (gr_line (start 121.5 123.5) (end 121.5 108) (stroke (width 0.05) (type default)) (layer "Edge.Cuts"))
 (gr_line (start 126 103.5) (end 154.5 103.5) (stroke (width 0.05) (type default)) (layer "Edge.Cuts"))
 (gr_arc (start 126 128) (mid 122.818019 126.681981) (end 121.5 123.5) (stroke (width 0.05) (type default)) (layer "Edge.Cuts"))
 (gr_line (start 126 128) (end 154.5 128) (stroke (width 0.05) (type default)) (layer "Edge.Cuts"))
 (gr_arc (start 154.5 103.5) (mid 157.681981 104.818019) (end 159 108) (stroke (width 0.05) (type default)) (layer "Edge.Cuts"))
 (gr_line (start 159 108) (end 159 123.5) (stroke (width 0.05) (type default)) (layer "Edge.Cuts"))
 (gr_arc (start 159 123.5) (mid 157.681981 126.681981) (end 154.5 128) (stroke (width 0.05) (type default)) (layer "Edge.Cuts"))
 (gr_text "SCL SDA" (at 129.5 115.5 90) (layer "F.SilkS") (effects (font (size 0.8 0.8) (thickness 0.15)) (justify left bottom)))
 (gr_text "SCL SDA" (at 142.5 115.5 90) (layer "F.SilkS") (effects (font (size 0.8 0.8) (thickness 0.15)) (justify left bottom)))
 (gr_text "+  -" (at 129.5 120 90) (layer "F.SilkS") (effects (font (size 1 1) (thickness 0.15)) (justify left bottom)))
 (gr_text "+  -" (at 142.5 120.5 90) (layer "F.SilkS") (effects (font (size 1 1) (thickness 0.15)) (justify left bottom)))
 (segment (start 132.06 119.25) (end 147.025 119.25) (width 0.5) (layer "F.Cu") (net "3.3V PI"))
 (segment (start 132 119.31) (end 132.06 119.25) (width 0.2) (layer "F.Cu") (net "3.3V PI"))
 (segment (start 147.005 114.23) (end 147.025 114.25) (width 0.2) (layer "F.Cu") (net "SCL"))
 (segment (start 132 114.23) (end 147.005 114.23) (width 0.5) (layer "F.Cu") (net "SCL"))
 (segment (start 146.965 111.69) (end 147.025 111.75) (width 0.2) (layer "F.Cu") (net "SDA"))
 (segment (start 132 111.69) (end 146.965 111.69) (width 0.5) (layer "F.Cu") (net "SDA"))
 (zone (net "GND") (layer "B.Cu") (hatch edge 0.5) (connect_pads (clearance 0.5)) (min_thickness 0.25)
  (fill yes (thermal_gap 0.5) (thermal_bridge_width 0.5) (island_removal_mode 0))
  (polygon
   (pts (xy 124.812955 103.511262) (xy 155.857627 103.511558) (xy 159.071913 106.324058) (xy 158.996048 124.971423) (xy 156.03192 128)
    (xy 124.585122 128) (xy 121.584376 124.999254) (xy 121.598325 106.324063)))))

